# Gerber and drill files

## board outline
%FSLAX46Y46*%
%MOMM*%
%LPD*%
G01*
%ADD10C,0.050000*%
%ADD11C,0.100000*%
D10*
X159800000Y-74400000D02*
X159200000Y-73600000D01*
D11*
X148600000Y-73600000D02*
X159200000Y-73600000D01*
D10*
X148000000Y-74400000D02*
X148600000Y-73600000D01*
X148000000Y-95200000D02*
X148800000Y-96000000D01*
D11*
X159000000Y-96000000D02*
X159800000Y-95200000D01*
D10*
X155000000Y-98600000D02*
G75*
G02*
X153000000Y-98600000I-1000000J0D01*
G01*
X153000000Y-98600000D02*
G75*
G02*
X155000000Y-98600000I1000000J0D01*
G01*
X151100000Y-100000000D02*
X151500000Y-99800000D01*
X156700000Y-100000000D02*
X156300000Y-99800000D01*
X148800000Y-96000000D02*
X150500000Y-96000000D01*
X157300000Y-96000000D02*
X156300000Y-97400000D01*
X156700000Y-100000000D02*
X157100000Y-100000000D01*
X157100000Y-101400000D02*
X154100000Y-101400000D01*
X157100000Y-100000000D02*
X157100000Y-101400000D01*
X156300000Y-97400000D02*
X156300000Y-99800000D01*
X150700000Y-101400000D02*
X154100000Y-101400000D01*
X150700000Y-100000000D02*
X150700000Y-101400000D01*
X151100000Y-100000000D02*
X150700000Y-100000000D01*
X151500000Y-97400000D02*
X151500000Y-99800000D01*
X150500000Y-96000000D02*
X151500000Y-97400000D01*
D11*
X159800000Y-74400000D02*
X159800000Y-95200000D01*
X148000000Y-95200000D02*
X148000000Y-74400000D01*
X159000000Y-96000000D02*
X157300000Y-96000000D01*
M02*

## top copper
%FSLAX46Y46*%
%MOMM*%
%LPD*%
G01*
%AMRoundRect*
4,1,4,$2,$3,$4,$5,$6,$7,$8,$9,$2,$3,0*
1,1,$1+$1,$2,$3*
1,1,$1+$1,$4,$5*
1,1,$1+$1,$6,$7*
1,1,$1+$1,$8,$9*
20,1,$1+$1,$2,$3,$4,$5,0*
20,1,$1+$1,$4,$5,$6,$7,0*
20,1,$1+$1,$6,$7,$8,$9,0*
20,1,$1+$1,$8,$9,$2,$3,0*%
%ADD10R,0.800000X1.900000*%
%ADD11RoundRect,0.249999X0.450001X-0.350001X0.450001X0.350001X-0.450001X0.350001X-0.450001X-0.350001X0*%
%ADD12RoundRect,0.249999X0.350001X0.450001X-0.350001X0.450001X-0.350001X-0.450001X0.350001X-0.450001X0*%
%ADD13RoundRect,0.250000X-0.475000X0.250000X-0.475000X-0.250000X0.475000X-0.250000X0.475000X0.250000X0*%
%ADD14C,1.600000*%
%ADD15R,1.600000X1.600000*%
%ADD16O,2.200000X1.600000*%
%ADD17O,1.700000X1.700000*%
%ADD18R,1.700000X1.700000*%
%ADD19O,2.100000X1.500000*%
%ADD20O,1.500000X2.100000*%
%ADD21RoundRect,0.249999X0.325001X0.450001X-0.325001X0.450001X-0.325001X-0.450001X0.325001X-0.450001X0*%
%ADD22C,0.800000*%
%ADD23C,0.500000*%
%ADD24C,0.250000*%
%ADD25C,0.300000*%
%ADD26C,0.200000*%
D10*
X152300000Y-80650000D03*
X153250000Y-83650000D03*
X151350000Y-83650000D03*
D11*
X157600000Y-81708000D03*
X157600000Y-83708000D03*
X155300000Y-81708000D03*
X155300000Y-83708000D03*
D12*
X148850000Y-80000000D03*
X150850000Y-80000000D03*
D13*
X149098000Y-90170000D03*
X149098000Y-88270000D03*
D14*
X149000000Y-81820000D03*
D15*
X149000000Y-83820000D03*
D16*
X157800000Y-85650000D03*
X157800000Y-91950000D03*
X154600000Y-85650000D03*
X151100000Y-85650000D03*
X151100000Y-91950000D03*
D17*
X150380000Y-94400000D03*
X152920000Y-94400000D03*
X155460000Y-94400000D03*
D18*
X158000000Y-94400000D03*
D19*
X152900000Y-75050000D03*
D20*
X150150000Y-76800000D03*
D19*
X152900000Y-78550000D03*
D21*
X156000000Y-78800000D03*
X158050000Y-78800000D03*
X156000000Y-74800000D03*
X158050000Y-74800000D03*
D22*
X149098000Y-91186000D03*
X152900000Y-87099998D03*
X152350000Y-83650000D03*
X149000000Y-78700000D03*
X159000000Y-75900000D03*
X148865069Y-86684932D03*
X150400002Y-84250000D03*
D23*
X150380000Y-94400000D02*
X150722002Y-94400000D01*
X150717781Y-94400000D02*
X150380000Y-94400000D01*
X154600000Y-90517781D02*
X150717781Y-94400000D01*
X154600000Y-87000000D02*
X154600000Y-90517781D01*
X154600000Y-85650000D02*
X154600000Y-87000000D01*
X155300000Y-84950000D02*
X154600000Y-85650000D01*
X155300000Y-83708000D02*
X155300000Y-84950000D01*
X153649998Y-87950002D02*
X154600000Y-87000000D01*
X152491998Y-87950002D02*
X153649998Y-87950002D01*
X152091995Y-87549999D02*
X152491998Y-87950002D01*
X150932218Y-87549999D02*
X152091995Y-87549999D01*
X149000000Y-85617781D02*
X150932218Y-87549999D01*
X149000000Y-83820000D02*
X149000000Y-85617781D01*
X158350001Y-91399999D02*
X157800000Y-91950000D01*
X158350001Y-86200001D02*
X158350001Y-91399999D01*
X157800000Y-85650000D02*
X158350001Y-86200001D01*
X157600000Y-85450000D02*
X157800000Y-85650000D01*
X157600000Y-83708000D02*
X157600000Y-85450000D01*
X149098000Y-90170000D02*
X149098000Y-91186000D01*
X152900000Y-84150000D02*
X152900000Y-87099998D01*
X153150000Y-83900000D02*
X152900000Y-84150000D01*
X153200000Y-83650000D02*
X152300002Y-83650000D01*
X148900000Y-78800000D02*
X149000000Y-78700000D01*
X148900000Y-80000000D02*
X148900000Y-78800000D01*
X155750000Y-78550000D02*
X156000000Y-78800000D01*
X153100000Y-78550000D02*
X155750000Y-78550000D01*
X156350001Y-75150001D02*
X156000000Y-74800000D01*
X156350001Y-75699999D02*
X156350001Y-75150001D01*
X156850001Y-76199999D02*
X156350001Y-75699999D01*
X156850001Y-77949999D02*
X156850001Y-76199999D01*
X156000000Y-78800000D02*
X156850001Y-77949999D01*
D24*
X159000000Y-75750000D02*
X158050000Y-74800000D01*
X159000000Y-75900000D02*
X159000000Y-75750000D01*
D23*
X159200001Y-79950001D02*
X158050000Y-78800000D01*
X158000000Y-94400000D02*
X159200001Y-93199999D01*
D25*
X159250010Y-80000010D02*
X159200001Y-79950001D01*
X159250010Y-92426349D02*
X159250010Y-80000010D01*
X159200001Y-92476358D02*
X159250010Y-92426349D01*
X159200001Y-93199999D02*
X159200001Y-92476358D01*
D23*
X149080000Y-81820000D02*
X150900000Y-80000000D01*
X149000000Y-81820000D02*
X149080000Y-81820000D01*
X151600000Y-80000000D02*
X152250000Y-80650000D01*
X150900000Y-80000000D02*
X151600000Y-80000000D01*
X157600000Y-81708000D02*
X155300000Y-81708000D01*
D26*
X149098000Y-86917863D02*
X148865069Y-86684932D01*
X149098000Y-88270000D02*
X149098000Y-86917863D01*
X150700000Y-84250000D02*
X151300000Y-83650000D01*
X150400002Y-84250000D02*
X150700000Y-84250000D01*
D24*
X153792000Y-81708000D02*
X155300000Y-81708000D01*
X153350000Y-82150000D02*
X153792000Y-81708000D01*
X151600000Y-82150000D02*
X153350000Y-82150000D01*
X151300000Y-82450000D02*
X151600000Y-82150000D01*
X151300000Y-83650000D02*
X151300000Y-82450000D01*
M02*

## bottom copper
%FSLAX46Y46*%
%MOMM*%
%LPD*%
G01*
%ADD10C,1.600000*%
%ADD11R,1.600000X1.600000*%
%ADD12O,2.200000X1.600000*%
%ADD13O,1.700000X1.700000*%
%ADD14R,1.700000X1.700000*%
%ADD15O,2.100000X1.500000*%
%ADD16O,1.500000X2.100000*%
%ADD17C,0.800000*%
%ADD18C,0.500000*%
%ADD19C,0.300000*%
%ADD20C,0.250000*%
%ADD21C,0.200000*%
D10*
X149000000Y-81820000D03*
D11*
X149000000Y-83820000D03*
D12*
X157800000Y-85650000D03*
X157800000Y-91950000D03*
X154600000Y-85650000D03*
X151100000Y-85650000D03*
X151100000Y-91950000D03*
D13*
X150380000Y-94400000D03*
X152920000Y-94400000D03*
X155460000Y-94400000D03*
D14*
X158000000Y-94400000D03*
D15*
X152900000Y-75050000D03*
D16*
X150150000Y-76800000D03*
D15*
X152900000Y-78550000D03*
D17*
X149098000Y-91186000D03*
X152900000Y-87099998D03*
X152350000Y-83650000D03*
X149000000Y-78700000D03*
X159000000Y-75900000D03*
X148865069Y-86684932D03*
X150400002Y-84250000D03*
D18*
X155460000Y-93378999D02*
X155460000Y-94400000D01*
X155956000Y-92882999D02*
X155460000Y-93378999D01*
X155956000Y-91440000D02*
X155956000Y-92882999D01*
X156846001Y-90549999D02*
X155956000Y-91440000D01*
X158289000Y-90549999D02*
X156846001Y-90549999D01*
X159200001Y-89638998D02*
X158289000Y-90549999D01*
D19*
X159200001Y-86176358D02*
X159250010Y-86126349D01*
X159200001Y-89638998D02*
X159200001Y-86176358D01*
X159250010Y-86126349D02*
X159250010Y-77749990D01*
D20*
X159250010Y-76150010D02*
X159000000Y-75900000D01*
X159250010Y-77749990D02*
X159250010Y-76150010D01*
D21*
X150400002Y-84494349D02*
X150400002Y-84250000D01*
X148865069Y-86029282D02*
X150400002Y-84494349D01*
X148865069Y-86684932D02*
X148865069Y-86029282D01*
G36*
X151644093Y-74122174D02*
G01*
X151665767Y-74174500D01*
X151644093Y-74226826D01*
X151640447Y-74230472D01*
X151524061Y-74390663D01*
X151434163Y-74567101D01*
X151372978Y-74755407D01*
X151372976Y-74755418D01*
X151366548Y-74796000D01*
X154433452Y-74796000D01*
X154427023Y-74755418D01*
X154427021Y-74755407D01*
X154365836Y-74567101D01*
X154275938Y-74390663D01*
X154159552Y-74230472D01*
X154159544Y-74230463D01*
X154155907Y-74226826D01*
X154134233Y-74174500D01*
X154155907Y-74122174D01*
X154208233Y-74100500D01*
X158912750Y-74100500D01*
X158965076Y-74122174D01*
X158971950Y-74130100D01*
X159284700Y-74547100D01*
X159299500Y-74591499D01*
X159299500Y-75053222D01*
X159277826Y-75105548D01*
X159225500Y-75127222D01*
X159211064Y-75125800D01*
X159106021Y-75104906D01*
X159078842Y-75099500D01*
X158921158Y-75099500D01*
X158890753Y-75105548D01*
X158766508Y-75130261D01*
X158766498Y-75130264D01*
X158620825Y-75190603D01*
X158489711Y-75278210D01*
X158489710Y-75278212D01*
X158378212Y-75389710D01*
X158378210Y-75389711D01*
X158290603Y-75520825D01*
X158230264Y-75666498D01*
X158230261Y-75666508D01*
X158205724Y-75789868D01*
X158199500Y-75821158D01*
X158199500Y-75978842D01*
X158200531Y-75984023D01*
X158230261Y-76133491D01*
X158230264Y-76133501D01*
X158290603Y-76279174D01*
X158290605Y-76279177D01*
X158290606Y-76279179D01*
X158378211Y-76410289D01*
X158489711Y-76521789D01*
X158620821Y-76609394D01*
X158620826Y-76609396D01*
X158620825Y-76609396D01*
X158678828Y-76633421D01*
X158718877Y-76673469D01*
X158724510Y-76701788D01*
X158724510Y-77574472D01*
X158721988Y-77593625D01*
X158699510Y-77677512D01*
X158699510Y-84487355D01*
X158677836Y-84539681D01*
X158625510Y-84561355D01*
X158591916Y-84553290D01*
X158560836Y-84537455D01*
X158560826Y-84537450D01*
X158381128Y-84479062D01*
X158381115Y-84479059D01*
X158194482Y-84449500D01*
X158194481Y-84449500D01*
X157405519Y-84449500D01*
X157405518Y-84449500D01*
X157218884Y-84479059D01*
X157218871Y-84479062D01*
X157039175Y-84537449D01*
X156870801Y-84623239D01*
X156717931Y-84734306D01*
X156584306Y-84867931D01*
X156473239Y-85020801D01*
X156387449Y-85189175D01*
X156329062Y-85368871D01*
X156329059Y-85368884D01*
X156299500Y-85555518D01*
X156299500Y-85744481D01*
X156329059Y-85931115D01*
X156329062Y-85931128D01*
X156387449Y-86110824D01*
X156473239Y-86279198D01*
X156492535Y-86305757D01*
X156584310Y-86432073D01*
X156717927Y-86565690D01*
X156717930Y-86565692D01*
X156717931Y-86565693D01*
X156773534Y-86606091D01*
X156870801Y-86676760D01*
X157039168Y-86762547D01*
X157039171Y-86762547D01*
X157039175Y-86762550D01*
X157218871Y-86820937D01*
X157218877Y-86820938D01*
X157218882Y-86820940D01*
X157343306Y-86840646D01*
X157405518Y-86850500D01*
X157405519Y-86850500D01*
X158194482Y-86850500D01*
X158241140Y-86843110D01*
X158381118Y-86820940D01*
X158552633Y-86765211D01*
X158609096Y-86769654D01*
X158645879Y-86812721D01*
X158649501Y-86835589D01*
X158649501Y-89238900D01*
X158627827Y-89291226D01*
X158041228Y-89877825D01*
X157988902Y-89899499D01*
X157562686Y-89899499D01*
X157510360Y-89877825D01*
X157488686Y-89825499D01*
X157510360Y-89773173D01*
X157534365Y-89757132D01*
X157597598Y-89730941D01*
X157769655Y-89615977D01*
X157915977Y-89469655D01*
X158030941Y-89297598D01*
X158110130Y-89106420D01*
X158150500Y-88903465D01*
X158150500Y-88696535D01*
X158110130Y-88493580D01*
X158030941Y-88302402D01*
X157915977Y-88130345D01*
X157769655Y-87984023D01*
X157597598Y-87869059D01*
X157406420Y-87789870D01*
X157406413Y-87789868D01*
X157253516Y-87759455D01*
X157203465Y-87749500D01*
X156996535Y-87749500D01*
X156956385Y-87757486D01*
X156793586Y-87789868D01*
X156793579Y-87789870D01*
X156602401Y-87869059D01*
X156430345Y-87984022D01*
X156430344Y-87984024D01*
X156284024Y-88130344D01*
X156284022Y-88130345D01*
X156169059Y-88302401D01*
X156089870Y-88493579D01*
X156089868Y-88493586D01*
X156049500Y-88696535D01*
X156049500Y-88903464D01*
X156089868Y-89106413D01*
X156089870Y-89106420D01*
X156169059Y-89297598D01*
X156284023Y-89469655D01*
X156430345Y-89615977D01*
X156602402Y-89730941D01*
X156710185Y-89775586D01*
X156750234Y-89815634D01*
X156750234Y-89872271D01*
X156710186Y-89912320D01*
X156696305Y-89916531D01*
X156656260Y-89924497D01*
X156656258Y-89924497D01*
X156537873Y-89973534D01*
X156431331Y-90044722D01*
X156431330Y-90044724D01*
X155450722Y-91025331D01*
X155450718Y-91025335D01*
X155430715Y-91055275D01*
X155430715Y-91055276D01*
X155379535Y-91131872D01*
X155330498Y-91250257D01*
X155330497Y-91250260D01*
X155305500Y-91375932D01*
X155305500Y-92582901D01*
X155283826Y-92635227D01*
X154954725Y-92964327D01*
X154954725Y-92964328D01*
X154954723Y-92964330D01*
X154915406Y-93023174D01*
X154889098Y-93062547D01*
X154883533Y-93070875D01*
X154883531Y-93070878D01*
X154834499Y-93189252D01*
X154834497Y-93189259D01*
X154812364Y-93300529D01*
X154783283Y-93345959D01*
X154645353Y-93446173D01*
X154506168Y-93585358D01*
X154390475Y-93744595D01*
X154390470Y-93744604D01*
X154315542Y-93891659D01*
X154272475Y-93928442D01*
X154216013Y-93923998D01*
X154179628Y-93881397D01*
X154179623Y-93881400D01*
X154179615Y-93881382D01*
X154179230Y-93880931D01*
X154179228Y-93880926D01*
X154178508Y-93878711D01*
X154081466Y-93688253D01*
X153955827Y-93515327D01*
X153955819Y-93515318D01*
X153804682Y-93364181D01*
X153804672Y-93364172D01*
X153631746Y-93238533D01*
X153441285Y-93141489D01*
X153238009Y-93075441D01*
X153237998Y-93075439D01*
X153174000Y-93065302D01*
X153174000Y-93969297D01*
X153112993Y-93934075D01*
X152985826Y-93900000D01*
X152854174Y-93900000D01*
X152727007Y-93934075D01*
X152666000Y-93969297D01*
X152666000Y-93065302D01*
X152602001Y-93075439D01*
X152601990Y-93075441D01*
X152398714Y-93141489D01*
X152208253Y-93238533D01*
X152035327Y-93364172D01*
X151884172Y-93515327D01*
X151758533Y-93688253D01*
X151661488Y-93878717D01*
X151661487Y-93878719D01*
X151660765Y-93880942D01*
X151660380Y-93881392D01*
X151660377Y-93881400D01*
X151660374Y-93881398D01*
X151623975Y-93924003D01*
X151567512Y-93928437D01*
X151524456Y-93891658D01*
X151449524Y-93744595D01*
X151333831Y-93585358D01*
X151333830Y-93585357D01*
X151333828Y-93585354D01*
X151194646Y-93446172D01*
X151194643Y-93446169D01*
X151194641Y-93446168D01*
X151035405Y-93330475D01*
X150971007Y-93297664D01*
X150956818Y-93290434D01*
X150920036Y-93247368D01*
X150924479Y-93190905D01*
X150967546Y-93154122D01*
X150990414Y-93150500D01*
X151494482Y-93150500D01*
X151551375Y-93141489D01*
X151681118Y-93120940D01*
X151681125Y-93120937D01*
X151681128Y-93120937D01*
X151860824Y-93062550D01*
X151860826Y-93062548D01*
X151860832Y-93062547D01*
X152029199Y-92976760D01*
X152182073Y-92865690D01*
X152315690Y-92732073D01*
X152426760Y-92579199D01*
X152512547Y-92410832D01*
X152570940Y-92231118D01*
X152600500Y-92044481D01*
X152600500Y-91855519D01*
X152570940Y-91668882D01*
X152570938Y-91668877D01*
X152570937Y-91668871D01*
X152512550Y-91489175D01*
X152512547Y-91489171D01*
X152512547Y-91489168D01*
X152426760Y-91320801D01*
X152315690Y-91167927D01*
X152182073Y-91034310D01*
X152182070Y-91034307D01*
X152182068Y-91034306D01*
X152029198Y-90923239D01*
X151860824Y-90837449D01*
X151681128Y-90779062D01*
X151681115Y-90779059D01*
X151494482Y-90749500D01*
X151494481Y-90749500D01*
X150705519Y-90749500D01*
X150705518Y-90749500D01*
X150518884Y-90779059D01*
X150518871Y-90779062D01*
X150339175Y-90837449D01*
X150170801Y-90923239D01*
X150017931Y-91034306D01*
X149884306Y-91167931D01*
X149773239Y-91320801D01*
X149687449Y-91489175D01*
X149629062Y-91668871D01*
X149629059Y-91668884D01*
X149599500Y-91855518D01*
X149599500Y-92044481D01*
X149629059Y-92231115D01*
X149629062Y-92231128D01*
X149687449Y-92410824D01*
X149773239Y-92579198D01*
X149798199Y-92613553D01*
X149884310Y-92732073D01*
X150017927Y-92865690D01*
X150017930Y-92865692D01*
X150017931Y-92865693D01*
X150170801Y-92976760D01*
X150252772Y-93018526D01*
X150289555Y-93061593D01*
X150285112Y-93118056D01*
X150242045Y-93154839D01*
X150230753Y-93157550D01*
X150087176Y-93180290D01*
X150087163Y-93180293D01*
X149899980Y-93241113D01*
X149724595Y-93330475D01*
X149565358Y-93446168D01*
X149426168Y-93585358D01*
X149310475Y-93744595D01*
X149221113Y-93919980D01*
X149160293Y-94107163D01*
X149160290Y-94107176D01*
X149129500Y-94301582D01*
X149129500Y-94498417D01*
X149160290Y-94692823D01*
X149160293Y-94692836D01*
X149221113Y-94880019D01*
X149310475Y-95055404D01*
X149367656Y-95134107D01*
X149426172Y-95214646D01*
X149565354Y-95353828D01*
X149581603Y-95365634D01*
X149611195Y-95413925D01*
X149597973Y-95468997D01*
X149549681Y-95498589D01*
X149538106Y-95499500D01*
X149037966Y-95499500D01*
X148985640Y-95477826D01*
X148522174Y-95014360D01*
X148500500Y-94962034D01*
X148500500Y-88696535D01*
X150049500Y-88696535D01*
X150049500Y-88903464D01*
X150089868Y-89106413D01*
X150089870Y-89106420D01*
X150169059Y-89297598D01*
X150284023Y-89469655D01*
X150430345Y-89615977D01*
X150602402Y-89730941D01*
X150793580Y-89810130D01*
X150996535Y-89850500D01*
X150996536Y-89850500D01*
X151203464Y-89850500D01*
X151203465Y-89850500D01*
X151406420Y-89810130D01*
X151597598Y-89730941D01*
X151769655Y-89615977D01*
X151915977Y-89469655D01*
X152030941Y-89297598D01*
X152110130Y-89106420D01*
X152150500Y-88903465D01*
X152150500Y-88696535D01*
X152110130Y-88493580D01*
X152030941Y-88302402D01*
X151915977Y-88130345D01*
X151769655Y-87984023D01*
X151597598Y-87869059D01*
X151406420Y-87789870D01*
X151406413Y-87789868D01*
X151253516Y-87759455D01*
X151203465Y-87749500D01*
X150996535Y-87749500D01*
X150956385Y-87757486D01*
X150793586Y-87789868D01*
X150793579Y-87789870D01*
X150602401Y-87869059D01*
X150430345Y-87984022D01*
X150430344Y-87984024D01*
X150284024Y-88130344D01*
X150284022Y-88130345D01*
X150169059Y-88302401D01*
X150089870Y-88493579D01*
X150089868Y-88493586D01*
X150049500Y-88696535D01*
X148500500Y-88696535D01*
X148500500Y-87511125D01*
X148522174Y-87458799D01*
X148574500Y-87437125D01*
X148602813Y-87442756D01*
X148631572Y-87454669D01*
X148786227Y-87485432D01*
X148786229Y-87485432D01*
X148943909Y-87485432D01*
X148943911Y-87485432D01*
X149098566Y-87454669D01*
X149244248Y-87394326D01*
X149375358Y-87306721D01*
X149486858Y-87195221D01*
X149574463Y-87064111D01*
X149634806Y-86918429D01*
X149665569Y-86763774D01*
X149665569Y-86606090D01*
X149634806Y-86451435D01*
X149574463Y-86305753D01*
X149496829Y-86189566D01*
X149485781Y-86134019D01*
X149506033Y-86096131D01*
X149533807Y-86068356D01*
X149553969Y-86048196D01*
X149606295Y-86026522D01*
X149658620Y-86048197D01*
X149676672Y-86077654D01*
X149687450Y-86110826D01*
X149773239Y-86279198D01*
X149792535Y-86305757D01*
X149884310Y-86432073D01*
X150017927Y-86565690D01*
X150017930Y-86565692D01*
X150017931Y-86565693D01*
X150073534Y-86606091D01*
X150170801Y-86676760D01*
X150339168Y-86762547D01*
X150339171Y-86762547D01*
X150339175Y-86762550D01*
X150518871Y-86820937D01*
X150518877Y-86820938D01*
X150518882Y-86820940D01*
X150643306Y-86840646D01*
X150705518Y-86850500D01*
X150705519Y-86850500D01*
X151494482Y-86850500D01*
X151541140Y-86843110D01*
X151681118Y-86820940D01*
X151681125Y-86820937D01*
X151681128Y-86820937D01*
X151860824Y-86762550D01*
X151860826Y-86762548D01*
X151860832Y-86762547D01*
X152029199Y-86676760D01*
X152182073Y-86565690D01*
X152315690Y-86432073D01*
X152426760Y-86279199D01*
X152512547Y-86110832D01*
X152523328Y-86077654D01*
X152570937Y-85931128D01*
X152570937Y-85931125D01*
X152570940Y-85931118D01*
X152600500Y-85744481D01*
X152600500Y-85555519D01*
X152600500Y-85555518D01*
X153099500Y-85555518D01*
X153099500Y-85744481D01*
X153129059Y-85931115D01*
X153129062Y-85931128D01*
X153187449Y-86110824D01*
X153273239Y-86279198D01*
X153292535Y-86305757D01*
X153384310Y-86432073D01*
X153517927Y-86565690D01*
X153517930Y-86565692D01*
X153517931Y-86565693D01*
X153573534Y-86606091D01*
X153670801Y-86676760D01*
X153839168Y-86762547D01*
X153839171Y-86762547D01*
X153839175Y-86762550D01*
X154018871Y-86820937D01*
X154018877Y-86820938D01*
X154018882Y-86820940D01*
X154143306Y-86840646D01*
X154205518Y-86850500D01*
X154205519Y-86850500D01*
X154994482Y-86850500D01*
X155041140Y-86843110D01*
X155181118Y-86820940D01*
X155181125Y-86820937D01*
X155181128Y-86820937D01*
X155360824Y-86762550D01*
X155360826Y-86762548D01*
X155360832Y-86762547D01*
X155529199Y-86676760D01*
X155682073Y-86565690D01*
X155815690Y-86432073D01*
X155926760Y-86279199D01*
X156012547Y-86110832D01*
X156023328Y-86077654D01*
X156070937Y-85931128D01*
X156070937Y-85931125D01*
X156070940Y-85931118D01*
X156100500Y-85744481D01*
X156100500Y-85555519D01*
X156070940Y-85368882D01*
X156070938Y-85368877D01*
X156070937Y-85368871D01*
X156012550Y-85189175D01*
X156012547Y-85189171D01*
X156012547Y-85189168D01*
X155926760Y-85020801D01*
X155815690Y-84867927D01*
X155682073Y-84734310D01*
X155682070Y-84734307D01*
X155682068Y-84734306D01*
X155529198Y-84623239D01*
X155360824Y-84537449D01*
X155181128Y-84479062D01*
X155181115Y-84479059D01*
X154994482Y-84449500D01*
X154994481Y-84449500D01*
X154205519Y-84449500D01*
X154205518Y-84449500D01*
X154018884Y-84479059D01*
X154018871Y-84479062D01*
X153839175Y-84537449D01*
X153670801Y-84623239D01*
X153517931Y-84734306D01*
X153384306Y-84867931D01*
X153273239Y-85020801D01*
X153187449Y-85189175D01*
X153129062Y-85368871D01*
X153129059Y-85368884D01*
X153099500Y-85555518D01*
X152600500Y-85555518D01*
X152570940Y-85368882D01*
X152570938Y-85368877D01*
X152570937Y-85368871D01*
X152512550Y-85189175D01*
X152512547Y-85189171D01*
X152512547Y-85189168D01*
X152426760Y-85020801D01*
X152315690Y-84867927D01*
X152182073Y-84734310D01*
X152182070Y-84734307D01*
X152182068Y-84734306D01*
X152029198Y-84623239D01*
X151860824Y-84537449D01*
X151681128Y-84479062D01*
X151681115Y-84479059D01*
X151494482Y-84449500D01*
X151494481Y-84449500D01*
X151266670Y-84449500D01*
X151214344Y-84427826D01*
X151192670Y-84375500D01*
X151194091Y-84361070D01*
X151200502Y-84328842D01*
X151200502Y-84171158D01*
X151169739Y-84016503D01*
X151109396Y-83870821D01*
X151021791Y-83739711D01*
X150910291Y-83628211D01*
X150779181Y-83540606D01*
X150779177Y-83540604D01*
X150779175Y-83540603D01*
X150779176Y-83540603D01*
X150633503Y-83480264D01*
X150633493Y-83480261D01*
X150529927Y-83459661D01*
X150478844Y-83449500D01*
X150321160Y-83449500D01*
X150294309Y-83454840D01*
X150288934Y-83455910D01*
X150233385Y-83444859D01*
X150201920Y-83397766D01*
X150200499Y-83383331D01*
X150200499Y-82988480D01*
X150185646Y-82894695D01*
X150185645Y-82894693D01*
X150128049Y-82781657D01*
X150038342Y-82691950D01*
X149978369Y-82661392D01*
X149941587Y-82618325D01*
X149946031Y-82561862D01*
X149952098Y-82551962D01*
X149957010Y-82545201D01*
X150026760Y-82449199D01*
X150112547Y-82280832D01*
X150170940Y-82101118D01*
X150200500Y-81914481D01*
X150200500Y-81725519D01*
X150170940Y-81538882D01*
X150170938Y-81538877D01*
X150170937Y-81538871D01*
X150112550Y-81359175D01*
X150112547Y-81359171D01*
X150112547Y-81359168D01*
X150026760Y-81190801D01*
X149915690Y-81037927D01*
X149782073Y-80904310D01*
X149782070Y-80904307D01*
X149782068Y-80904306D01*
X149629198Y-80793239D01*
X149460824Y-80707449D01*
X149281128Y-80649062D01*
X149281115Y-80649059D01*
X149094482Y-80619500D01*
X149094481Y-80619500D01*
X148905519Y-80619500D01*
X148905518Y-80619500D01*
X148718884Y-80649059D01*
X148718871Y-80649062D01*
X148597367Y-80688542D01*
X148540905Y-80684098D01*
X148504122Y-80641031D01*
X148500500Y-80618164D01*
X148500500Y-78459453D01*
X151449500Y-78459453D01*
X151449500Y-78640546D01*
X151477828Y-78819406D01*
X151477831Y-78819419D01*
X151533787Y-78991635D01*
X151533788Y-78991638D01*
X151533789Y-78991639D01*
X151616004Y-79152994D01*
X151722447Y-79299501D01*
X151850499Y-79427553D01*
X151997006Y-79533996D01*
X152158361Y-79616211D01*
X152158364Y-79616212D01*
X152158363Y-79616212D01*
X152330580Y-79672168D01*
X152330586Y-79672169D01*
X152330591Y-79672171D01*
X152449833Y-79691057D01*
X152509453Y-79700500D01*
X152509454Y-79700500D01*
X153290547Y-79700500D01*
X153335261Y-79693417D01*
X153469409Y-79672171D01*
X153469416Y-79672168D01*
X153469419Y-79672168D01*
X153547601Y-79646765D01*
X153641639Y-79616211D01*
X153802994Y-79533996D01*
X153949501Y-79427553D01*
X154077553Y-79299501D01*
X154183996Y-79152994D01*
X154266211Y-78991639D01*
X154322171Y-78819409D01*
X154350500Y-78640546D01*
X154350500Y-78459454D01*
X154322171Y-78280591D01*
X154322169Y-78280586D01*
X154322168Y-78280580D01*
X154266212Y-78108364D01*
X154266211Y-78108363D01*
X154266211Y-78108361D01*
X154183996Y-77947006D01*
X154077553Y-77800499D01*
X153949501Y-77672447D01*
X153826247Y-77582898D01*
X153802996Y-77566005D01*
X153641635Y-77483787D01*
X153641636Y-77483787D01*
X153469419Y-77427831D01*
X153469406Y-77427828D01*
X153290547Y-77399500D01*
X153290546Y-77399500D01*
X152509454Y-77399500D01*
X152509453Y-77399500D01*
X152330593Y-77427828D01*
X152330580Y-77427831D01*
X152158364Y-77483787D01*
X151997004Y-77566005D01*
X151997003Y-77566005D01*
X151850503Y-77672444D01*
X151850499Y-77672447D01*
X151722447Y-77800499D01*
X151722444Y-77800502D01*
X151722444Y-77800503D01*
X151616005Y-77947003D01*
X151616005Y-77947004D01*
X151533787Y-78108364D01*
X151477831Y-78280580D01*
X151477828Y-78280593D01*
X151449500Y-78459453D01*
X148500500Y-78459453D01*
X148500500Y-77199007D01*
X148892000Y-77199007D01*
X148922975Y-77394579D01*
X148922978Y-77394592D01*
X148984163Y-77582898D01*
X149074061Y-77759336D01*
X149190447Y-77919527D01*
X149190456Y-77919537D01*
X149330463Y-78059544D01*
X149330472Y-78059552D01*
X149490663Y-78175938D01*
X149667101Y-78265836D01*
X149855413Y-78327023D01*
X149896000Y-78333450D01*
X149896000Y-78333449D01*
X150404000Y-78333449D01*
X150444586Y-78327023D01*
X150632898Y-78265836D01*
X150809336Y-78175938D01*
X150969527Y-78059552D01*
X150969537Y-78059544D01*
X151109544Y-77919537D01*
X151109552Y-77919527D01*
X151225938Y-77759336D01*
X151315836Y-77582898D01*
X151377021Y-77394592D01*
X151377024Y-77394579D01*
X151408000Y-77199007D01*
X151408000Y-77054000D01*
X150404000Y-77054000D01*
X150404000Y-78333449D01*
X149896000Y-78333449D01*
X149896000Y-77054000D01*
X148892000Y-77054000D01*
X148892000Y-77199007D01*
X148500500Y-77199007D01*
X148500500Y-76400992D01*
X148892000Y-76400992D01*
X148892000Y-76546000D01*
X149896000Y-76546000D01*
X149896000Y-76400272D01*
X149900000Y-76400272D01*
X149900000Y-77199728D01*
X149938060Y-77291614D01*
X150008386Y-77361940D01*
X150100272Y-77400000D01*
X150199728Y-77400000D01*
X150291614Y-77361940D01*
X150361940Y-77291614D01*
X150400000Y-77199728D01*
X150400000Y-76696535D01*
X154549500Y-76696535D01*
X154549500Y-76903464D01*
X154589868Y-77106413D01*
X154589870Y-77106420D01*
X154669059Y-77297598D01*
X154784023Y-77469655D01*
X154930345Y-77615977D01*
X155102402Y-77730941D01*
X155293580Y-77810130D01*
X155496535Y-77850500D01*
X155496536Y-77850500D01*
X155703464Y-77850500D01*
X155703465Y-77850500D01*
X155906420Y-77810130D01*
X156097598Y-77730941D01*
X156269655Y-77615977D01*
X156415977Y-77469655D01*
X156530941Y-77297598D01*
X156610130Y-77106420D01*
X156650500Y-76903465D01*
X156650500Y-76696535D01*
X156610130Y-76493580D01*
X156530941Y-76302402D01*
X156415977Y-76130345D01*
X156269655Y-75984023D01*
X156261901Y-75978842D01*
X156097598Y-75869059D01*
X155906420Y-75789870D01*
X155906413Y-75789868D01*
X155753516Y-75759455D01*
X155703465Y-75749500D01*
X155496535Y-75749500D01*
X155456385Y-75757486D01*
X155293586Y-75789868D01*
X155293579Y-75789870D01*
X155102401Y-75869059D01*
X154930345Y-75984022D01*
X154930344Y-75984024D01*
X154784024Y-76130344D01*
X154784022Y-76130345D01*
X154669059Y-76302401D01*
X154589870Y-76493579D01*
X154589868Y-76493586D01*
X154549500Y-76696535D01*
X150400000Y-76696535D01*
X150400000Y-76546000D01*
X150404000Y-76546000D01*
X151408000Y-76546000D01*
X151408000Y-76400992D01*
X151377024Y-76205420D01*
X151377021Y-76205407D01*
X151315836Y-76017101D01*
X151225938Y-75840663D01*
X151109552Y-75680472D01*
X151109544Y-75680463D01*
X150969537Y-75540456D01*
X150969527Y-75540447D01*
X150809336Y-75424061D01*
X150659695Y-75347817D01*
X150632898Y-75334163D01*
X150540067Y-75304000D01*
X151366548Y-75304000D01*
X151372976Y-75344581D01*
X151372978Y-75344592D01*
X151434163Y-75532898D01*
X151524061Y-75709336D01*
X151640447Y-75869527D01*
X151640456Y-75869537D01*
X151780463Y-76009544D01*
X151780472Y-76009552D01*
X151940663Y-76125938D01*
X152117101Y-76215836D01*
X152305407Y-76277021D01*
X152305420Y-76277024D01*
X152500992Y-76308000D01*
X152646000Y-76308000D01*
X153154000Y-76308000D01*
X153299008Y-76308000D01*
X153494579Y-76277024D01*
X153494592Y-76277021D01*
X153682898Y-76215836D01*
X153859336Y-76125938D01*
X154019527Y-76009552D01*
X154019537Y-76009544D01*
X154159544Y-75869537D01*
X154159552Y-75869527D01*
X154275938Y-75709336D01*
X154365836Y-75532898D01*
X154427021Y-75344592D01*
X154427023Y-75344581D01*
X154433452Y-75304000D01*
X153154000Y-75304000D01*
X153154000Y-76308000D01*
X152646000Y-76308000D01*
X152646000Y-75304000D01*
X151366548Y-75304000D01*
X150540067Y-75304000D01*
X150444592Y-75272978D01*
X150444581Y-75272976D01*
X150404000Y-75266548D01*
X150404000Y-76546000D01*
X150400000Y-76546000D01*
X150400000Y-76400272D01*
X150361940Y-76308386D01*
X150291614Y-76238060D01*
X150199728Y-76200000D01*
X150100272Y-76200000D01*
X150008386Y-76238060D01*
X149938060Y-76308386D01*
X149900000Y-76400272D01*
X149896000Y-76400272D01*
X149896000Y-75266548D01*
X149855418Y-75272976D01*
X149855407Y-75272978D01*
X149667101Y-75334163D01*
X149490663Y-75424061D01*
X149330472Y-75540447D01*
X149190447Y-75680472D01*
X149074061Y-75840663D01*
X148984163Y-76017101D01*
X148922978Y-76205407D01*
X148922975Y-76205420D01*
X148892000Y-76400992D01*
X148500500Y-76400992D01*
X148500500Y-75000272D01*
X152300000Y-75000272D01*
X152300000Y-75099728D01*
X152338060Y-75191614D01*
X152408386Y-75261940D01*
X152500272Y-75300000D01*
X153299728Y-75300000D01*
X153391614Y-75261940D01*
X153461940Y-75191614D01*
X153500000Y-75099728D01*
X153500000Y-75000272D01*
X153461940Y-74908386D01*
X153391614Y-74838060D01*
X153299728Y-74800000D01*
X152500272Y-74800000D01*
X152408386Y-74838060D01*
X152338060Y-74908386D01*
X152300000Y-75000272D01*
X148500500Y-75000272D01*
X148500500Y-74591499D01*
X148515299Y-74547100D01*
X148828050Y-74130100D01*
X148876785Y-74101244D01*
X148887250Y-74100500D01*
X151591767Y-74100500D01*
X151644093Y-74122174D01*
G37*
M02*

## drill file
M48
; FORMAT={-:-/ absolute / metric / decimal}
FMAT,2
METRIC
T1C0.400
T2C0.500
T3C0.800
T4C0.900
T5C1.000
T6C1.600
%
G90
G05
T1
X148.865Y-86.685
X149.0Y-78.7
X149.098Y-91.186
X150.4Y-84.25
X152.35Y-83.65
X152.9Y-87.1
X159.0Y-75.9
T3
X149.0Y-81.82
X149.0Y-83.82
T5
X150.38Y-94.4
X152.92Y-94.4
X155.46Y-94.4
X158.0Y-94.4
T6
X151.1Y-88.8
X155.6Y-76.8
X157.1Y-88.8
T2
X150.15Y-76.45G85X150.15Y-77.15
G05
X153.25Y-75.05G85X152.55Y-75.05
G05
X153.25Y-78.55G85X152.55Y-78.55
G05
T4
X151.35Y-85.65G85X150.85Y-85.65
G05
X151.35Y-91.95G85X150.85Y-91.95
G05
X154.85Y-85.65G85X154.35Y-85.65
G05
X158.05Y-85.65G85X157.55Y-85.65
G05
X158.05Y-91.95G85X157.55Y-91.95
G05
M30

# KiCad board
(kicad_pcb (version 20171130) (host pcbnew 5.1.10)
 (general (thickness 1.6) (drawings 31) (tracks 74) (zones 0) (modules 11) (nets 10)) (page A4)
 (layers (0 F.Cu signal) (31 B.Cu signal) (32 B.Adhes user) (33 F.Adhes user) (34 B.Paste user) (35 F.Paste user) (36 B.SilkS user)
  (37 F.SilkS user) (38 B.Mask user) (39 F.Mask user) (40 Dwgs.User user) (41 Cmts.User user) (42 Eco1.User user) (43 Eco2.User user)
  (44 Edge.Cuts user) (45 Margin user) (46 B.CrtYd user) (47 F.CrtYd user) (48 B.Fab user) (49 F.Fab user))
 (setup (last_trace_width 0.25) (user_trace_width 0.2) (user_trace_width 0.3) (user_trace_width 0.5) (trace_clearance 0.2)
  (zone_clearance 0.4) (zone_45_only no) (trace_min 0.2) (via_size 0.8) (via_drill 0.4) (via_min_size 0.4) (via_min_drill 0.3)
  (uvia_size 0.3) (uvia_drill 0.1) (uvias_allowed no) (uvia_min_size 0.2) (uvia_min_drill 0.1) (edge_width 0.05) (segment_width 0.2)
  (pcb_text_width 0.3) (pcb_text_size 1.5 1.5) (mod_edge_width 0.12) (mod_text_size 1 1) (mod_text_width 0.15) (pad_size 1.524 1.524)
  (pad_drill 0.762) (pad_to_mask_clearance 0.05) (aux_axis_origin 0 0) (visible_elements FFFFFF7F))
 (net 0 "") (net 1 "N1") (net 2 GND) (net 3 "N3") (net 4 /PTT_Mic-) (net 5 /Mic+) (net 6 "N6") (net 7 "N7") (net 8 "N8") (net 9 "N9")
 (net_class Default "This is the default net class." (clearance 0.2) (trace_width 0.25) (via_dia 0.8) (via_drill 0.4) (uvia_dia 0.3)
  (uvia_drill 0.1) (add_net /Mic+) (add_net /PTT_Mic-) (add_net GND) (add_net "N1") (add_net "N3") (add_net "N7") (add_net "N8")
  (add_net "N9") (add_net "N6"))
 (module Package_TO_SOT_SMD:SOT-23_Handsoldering (layer F.Cu) (at 152.3 82.15 90)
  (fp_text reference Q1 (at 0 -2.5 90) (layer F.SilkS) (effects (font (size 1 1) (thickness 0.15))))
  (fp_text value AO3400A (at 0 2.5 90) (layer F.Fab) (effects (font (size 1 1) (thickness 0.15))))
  (pad 3 smd rect (at 1.5 0 90) (size 1.9 0.8) (layers F.Cu F.Paste F.Mask) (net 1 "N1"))
  (pad 2 smd rect (at -1.5 0.95 90) (size 1.9 0.8) (layers F.Cu F.Paste F.Mask) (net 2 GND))
  (pad 1 smd rect (at -1.5 -0.95 90) (size 1.9 0.8) (layers F.Cu F.Paste F.Mask) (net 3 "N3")))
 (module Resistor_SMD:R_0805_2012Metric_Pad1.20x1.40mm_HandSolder (layer F.Cu) (at 157.6 82.708 90)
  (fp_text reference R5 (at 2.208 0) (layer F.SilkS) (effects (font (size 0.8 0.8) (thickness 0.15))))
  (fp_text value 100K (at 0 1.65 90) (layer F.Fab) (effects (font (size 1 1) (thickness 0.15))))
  (pad 2 smd roundrect (at 1 0 90) (size 1.2 1.4) (layers F.Cu F.Paste F.Mask) (roundrect_rratio 0.2083325) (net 3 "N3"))
  (pad 1 smd roundrect (at -1 0 90) (size 1.2 1.4) (layers F.Cu F.Paste F.Mask) (roundrect_rratio 0.2083325) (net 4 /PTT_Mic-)))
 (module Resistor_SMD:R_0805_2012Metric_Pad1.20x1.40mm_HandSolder (layer F.Cu) (at 155.3 82.708 90)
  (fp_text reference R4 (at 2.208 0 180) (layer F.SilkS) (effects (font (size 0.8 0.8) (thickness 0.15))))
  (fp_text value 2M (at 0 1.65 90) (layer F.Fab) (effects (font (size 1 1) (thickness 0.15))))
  (pad 2 smd roundrect (at 1 0 90) (size 1.2 1.4) (layers F.Cu F.Paste F.Mask) (roundrect_rratio 0.2083325) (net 3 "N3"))
  (pad 1 smd roundrect (at -1 0 90) (size 1.2 1.4) (layers F.Cu F.Paste F.Mask) (roundrect_rratio 0.2083325) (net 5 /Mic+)))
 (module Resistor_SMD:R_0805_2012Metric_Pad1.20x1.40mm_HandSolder (layer F.Cu) (at 149.85 80 180)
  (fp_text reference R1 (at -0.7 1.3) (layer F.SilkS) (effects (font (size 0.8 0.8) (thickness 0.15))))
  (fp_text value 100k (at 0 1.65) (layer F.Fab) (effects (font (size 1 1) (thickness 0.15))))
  (pad 2 smd roundrect (at 1 0 180) (size 1.2 1.4) (layers F.Cu F.Paste F.Mask) (roundrect_rratio 0.2083325) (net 2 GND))
  (pad 1 smd roundrect (at -1 0 180) (size 1.2 1.4) (layers F.Cu F.Paste F.Mask) (roundrect_rratio 0.2083325) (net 1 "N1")))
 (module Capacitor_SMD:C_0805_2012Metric (layer F.Cu) (at 149.098 89.22 270)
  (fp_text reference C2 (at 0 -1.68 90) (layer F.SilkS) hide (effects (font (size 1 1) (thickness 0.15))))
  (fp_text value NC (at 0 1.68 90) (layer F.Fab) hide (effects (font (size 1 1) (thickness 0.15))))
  (pad 2 smd roundrect (at 0.95 0 270) (size 1 1.45) (layers F.Cu F.Paste F.Mask) (roundrect_rratio 0.25) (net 2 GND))
  (pad 1 smd roundrect (at -0.95 0 270) (size 1 1.45) (layers F.Cu F.Paste F.Mask) (roundrect_rratio 0.25) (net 3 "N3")))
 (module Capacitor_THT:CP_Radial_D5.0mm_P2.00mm (layer B.Cu) (at 149 83.82 90)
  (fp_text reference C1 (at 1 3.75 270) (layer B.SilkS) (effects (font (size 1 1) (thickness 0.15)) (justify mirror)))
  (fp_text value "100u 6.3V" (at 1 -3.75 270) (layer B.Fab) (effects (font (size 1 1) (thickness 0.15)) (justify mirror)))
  (pad 2 thru_hole circle (at 2 0 90) (size 1.6 1.6) (drill 0.8) (layers *.Cu *.Mask) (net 1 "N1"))
  (pad 1 thru_hole rect (at 0 0 90) (size 1.6 1.6) (drill 0.8) (layers *.Cu *.Mask) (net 5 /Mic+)))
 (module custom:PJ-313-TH (layer B.Cu) (at 159.6 88.8 180)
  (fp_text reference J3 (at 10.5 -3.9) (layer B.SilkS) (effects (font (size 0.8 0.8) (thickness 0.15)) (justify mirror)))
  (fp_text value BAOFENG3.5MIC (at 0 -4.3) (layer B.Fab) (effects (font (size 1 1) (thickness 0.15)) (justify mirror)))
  (pad "" np_thru_hole circle (at 2.5 0 180) (size 1.6 1.6) (drill 1.6) (layers *.Cu *.Mask))
  (pad "" np_thru_hole circle (at 8.5 0 180) (size 1.6 1.6) (drill 1.6) (layers *.Cu *.Mask))
  (pad S thru_hole oval (at 1.8 3.15 180) (size 2.2 1.6) (drill oval 1.4 0.9) (layers *.Cu *.Mask) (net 4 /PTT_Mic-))
  (pad S thru_hole oval (at 1.8 -3.15 180) (size 2.2 1.6) (drill oval 1.4 0.9) (layers *.Cu *.Mask) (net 4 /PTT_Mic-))
  (pad R thru_hole oval (at 5 3.15 180) (size 2.2 1.6) (drill oval 1.4 0.9) (layers *.Cu *.Mask) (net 5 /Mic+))
  (pad T thru_hole oval (at 8.5 3.15 180) (size 2.2 1.6) (drill oval 1.4 0.9) (layers *.Cu *.Mask) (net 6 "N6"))
  (pad T thru_hole oval (at 8.5 -3.15 180) (size 2.2 1.6) (drill oval 1.4 0.9) (layers *.Cu *.Mask) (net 6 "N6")))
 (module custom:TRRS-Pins (layer F.Cu) (at 158 94.4 270)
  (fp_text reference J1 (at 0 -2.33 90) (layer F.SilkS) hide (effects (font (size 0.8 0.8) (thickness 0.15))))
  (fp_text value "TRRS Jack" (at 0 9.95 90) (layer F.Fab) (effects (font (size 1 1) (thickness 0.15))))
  (pad S thru_hole oval (at 0 7.62 270) (size 1.7 1.7) (drill 1) (layers *.Cu *.Mask) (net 5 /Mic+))
  (pad R2 thru_hole oval (at 0 5.08 270) (size 1.7 1.7) (drill 1) (layers *.Cu *.Mask) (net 2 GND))
  (pad R1 thru_hole oval (at 0 2.54 270) (size 1.7 1.7) (drill 1) (layers *.Cu *.Mask) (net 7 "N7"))
  (pad T thru_hole rect (at 0 0 270) (size 1.7 1.7) (drill 1) (layers *.Cu *.Mask) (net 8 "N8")))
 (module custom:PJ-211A (layer B.Cu) (at 159.1 76.8 270)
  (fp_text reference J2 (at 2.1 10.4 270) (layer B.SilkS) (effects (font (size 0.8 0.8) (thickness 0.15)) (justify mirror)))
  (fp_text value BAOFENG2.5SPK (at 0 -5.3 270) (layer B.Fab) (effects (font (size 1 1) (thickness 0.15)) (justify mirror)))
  (pad R thru_hole oval (at -1.75 6.2 270) (size 1.5 2.1) (drill oval 0.5 1.2) (layers *.Cu *.Mask) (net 2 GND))
  (pad S thru_hole oval (at 0 8.95 270) (size 2.1 1.5) (drill oval 1.2 0.5) (layers *.Cu *.Mask) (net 2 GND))
  (pad T thru_hole oval (at 1.75 6.2 270) (size 1.5 2.1) (drill oval 0.5 1.2) (layers *.Cu *.Mask) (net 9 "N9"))
  (pad "" np_thru_hole circle (at 0 3.5 270) (size 1.6 1.6) (drill 1.6) (layers *.Cu *.Mask)))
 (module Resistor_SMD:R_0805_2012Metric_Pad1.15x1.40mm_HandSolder (layer F.Cu) (at 157.025 78.8 180)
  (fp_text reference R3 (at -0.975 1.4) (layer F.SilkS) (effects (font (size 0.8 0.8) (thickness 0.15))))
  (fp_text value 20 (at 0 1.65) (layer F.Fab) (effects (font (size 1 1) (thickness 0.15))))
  (pad 2 smd roundrect (at 1.025 0 180) (size 1.15 1.4) (layers F.Cu F.Paste F.Mask) (roundrect_rratio 0.2173904347826087) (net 9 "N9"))
  (pad 1 smd roundrect (at -1.025 0 180) (size 1.15 1.4) (layers F.Cu F.Paste F.Mask) (roundrect_rratio 0.2173904347826087) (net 8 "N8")))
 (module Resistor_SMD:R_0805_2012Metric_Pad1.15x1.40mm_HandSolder (layer F.Cu) (at 157.025 74.8 180)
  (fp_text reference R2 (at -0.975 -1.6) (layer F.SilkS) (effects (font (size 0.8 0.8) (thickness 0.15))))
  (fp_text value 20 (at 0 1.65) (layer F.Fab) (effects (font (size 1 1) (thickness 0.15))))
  (pad 2 smd roundrect (at 1.025 0 180) (size 1.15 1.4) (layers F.Cu F.Paste F.Mask) (roundrect_rratio 0.2173904347826087) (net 9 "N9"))
  (pad 1 smd roundrect (at -1.025 0 180) (size 1.15 1.4) (layers F.Cu F.Paste F.Mask) (roundrect_rratio 0.2173904347826087) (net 7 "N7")))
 (gr_line (start 159.8 74.4) (end 159.2 73.6) (layer Edge.Cuts) (width 0.05))
 (gr_line (start 148.6 73.6) (end 159.2 73.6) (layer Edge.Cuts) (width 0.1))
 (gr_line (start 148 74.4) (end 148.6 73.6) (layer Edge.Cuts) (width 0.05))
 (gr_line (start 148 95.2) (end 148.8 96) (layer Edge.Cuts) (width 0.05))
 (gr_line (start 159 96) (end 159.8 95.2) (layer Edge.Cuts) (width 0.1))
 (gr_circle (center 154 98.6) (end 155 98.6) (layer Edge.Cuts) (width 0.05))
 (gr_line (start 151.1 100) (end 151.5 99.8) (layer Edge.Cuts) (width 0.05))
 (gr_line (start 156.7 100) (end 156.3 99.8) (layer Edge.Cuts) (width 0.05))
 (gr_line (start 148.8 96) (end 150.5 96) (layer Edge.Cuts) (width 0.05))
 (gr_line (start 157.3 96) (end 156.3 97.4) (layer Edge.Cuts) (width 0.05))
 (gr_line (start 156.7 100) (end 157.1 100) (layer Edge.Cuts) (width 0.05))
 (gr_line (start 157.1 101.4) (end 154.1 101.4) (layer Edge.Cuts) (width 0.05))
 (gr_line (start 157.1 100) (end 157.1 101.4) (layer Edge.Cuts) (width 0.05))
 (gr_line (start 156.3 97.4) (end 156.3 99.8) (layer Edge.Cuts) (width 0.05))
 (gr_line (start 150.7 101.4) (end 154.1 101.4) (layer Edge.Cuts) (width 0.05))
 (gr_line (start 150.7 100) (end 150.7 101.4) (layer Edge.Cuts) (width 0.05))
 (gr_line (start 151.1 100) (end 150.7 100) (layer Edge.Cuts) (width 0.05))
 (gr_line (start 151.5 97.4) (end 151.5 99.8) (layer Edge.Cuts) (width 0.05))
 (gr_line (start 150.5 96) (end 151.5 97.4) (layer Edge.Cuts) (width 0.05))
 (gr_line (start 159.8 74.4) (end 159.8 95.2) (layer Edge.Cuts) (width 0.1))
 (gr_line (start 148 95.2) (end 148 74.4) (layer Edge.Cuts) (width 0.1))
 (gr_line (start 159 96) (end 157.3 96) (layer Edge.Cuts) (width 0.1))
 (segment (start 150.38 94.4) (end 150.722002 94.4) (width 0.5) (layer F.Cu) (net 5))
 (segment (start 150.717781 94.4) (end 150.38 94.4) (width 0.5) (layer F.Cu) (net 5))
 (segment (start 154.6 90.517781) (end 150.717781 94.4) (width 0.5) (layer F.Cu) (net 5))
 (segment (start 154.6 87) (end 154.6 90.517781) (width 0.5) (layer F.Cu) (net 5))
 (segment (start 154.6 85.65) (end 154.6 87) (width 0.5) (layer F.Cu) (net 5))
 (segment (start 155.3 84.95) (end 154.6 85.65) (width 0.5) (layer F.Cu) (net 5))
 (segment (start 155.3 83.708) (end 155.3 84.95) (width 0.5) (layer F.Cu) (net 5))
 (segment (start 153.649998 87.950002) (end 154.6 87) (width 0.5) (layer F.Cu) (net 5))
 (segment (start 152.491998 87.950002) (end 153.649998 87.950002) (width 0.5) (layer F.Cu) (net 5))
 (segment (start 152.091995 87.549999) (end 152.491998 87.950002) (width 0.5) (layer F.Cu) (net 5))
 (segment (start 150.932218 87.549999) (end 152.091995 87.549999) (width 0.5) (layer F.Cu) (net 5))
 (segment (start 149 85.617781) (end 150.932218 87.549999) (width 0.5) (layer F.Cu) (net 5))
 (segment (start 149 83.82) (end 149 85.617781) (width 0.5) (layer F.Cu) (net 5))
 (segment (start 158.350001 91.399999) (end 157.8 91.95) (width 0.5) (layer F.Cu) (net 4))
 (segment (start 158.350001 86.200001) (end 158.350001 91.399999) (width 0.5) (layer F.Cu) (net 4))
 (segment (start 157.8 85.65) (end 158.350001 86.200001) (width 0.5) (layer F.Cu) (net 4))
 (segment (start 157.6 85.45) (end 157.8 85.65) (width 0.5) (layer F.Cu) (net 4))
 (segment (start 157.6 83.708) (end 157.6 85.45) (width 0.5) (layer F.Cu) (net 4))
 (via (at 149.098 91.186) (size 0.8) (drill 0.4) (layers F.Cu B.Cu) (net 2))
 (segment (start 149.098 90.17) (end 149.098 91.186) (width 0.5) (layer F.Cu) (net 2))
 (segment (start 152.9 84.15) (end 152.9 87.099998) (width 0.5) (layer F.Cu) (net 2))
 (via (at 152.9 87.099998) (size 0.8) (drill 0.4) (layers F.Cu B.Cu) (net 2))
 (segment (start 153.15 83.9) (end 152.9 84.15) (width 0.5) (layer F.Cu) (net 2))
 (via (at 152.35 83.65) (size 0.8) (drill 0.4) (layers F.Cu B.Cu) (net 2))
 (segment (start 153.2 83.65) (end 152.300002 83.65) (width 0.5) (layer F.Cu) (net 2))
 (via (at 149 78.7) (size 0.8) (drill 0.4) (layers F.Cu B.Cu) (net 2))
 (segment (start 148.9 78.8) (end 149 78.7) (width 0.5) (layer F.Cu) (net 2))
 (segment (start 148.9 80) (end 148.9 78.8) (width 0.5) (layer F.Cu) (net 2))
 (segment (start 155.75 78.55) (end 156 78.8) (width 0.5) (layer F.Cu) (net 9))
 (segment (start 153.1 78.55) (end 155.75 78.55) (width 0.5) (layer F.Cu) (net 9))
 (segment (start 156.350001 75.150001) (end 156 74.8) (width 0.5) (layer F.Cu) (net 9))
 (segment (start 156.350001 75.699999) (end 156.350001 75.150001) (width 0.5) (layer F.Cu) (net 9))
 (segment (start 156.850001 76.199999) (end 156.350001 75.699999) (width 0.5) (layer F.Cu) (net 9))
 (segment (start 156.850001 77.949999) (end 156.850001 76.199999) (width 0.5) (layer F.Cu) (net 9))
 (segment (start 156 78.8) (end 156.850001 77.949999) (width 0.5) (layer F.Cu) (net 9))
 (segment (start 155.46 93.378999) (end 155.46 94.4) (width 0.5) (layer B.Cu) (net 7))
 (segment (start 155.956 92.882999) (end 155.46 93.378999) (width 0.5) (layer B.Cu) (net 7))
 (segment (start 155.956 91.44) (end 155.956 92.882999) (width 0.5) (layer B.Cu) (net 7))
 (segment (start 156.846001 90.549999) (end 155.956 91.44) (width 0.5) (layer B.Cu) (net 7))
 (segment (start 158.289 90.549999) (end 156.846001 90.549999) (width 0.5) (layer B.Cu) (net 7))
 (segment (start 159.200001 89.638998) (end 158.289 90.549999) (width 0.5) (layer B.Cu) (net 7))
 (segment (start 159.200001 86.176358) (end 159.25001 86.126349) (width 0.3) (layer B.Cu) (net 7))
 (segment (start 159.200001 89.638998) (end 159.200001 86.176358) (width 0.3) (layer B.Cu) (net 7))
 (segment (start 159.25001 86.126349) (end 159.25001 77.74999) (width 0.3) (layer B.Cu) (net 7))
 (via (at 159 75.9) (size 0.8) (drill 0.4) (layers F.Cu B.Cu) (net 7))
 (segment (start 159.25001 76.15001) (end 159 75.9) (width 0.25) (layer B.Cu) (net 7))
 (segment (start 159.25001 77.74999) (end 159.25001 76.15001) (width 0.25) (layer B.Cu) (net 7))
 (segment (start 159 75.75) (end 158.05 74.8) (width 0.25) (layer F.Cu) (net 7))
 (segment (start 159 75.9) (end 159 75.75) (width 0.25) (layer F.Cu) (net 7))
 (segment (start 159.200001 79.950001) (end 158.05 78.8) (width 0.5) (layer F.Cu) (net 8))
 (segment (start 158 94.4) (end 159.200001 93.199999) (width 0.5) (layer F.Cu) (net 8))
 (segment (start 159.25001 80.00001) (end 159.200001 79.950001) (width 0.3) (layer F.Cu) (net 8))
 (segment (start 159.25001 92.426349) (end 159.25001 80.00001) (width 0.3) (layer F.Cu) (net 8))
 (segment (start 159.200001 92.476358) (end 159.25001 92.426349) (width 0.3) (layer F.Cu) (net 8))
 (segment (start 159.200001 93.199999) (end 159.200001 92.476358) (width 0.3) (layer F.Cu) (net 8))
 (segment (start 149.08 81.82) (end 150.9 80) (width 0.5) (layer F.Cu) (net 1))
 (segment (start 149 81.82) (end 149.08 81.82) (width 0.5) (layer F.Cu) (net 1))
 (segment (start 151.6 80) (end 152.25 80.65) (width 0.5) (layer F.Cu) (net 1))
 (segment (start 150.9 80) (end 151.6 80) (width 0.5) (layer F.Cu) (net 1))
 (segment (start 157.6 81.708) (end 155.3 81.708) (width 0.5) (layer F.Cu) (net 3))
 (via (at 148.865069 86.684932) (size 0.8) (drill 0.4) (layers F.Cu B.Cu) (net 3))
 (segment (start 149.098 86.917863) (end 148.865069 86.684932) (width 0.2) (layer F.Cu) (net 3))
 (segment (start 149.098 88.27) (end 149.098 86.917863) (width 0.2) (layer F.Cu) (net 3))
 (via (at 150.400002 84.25) (size 0.8) (drill 0.4) (layers F.Cu B.Cu) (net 3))
 (segment (start 150.400002 84.494349) (end 150.400002 84.25) (width 0.2) (layer B.Cu) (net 3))
 (segment (start 148.865069 86.029282) (end 150.400002 84.494349) (width 0.2) (layer B.Cu) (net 3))
 (segment (start 148.865069 86.684932) (end 148.865069 86.029282) (width 0.2) (layer B.Cu) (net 3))
 (segment (start 150.7 84.25) (end 151.3 83.65) (width 0.2) (layer F.Cu) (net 3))
 (segment (start 150.400002 84.25) (end 150.7 84.25) (width 0.2) (layer F.Cu) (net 3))
 (segment (start 153.792 81.708) (end 155.3 81.708) (width 0.25) (layer F.Cu) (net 3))
 (segment (start 153.35 82.15) (end 153.792 81.708) (width 0.25) (layer F.Cu) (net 3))
 (segment (start 151.6 82.15) (end 153.35 82.15) (width 0.25) (layer F.Cu) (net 3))
 (segment (start 151.3 82.45) (end 151.6 82.15) (width 0.25) (layer F.Cu) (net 3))
 (segment (start 151.3 83.65) (end 151.3 82.45) (width 0.25) (layer F.Cu) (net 3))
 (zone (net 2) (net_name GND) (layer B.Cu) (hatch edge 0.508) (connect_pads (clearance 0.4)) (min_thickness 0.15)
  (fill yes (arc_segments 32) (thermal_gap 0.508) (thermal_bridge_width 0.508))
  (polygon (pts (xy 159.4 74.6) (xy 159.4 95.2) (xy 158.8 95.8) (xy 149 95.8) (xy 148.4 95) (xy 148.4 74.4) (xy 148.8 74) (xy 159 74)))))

